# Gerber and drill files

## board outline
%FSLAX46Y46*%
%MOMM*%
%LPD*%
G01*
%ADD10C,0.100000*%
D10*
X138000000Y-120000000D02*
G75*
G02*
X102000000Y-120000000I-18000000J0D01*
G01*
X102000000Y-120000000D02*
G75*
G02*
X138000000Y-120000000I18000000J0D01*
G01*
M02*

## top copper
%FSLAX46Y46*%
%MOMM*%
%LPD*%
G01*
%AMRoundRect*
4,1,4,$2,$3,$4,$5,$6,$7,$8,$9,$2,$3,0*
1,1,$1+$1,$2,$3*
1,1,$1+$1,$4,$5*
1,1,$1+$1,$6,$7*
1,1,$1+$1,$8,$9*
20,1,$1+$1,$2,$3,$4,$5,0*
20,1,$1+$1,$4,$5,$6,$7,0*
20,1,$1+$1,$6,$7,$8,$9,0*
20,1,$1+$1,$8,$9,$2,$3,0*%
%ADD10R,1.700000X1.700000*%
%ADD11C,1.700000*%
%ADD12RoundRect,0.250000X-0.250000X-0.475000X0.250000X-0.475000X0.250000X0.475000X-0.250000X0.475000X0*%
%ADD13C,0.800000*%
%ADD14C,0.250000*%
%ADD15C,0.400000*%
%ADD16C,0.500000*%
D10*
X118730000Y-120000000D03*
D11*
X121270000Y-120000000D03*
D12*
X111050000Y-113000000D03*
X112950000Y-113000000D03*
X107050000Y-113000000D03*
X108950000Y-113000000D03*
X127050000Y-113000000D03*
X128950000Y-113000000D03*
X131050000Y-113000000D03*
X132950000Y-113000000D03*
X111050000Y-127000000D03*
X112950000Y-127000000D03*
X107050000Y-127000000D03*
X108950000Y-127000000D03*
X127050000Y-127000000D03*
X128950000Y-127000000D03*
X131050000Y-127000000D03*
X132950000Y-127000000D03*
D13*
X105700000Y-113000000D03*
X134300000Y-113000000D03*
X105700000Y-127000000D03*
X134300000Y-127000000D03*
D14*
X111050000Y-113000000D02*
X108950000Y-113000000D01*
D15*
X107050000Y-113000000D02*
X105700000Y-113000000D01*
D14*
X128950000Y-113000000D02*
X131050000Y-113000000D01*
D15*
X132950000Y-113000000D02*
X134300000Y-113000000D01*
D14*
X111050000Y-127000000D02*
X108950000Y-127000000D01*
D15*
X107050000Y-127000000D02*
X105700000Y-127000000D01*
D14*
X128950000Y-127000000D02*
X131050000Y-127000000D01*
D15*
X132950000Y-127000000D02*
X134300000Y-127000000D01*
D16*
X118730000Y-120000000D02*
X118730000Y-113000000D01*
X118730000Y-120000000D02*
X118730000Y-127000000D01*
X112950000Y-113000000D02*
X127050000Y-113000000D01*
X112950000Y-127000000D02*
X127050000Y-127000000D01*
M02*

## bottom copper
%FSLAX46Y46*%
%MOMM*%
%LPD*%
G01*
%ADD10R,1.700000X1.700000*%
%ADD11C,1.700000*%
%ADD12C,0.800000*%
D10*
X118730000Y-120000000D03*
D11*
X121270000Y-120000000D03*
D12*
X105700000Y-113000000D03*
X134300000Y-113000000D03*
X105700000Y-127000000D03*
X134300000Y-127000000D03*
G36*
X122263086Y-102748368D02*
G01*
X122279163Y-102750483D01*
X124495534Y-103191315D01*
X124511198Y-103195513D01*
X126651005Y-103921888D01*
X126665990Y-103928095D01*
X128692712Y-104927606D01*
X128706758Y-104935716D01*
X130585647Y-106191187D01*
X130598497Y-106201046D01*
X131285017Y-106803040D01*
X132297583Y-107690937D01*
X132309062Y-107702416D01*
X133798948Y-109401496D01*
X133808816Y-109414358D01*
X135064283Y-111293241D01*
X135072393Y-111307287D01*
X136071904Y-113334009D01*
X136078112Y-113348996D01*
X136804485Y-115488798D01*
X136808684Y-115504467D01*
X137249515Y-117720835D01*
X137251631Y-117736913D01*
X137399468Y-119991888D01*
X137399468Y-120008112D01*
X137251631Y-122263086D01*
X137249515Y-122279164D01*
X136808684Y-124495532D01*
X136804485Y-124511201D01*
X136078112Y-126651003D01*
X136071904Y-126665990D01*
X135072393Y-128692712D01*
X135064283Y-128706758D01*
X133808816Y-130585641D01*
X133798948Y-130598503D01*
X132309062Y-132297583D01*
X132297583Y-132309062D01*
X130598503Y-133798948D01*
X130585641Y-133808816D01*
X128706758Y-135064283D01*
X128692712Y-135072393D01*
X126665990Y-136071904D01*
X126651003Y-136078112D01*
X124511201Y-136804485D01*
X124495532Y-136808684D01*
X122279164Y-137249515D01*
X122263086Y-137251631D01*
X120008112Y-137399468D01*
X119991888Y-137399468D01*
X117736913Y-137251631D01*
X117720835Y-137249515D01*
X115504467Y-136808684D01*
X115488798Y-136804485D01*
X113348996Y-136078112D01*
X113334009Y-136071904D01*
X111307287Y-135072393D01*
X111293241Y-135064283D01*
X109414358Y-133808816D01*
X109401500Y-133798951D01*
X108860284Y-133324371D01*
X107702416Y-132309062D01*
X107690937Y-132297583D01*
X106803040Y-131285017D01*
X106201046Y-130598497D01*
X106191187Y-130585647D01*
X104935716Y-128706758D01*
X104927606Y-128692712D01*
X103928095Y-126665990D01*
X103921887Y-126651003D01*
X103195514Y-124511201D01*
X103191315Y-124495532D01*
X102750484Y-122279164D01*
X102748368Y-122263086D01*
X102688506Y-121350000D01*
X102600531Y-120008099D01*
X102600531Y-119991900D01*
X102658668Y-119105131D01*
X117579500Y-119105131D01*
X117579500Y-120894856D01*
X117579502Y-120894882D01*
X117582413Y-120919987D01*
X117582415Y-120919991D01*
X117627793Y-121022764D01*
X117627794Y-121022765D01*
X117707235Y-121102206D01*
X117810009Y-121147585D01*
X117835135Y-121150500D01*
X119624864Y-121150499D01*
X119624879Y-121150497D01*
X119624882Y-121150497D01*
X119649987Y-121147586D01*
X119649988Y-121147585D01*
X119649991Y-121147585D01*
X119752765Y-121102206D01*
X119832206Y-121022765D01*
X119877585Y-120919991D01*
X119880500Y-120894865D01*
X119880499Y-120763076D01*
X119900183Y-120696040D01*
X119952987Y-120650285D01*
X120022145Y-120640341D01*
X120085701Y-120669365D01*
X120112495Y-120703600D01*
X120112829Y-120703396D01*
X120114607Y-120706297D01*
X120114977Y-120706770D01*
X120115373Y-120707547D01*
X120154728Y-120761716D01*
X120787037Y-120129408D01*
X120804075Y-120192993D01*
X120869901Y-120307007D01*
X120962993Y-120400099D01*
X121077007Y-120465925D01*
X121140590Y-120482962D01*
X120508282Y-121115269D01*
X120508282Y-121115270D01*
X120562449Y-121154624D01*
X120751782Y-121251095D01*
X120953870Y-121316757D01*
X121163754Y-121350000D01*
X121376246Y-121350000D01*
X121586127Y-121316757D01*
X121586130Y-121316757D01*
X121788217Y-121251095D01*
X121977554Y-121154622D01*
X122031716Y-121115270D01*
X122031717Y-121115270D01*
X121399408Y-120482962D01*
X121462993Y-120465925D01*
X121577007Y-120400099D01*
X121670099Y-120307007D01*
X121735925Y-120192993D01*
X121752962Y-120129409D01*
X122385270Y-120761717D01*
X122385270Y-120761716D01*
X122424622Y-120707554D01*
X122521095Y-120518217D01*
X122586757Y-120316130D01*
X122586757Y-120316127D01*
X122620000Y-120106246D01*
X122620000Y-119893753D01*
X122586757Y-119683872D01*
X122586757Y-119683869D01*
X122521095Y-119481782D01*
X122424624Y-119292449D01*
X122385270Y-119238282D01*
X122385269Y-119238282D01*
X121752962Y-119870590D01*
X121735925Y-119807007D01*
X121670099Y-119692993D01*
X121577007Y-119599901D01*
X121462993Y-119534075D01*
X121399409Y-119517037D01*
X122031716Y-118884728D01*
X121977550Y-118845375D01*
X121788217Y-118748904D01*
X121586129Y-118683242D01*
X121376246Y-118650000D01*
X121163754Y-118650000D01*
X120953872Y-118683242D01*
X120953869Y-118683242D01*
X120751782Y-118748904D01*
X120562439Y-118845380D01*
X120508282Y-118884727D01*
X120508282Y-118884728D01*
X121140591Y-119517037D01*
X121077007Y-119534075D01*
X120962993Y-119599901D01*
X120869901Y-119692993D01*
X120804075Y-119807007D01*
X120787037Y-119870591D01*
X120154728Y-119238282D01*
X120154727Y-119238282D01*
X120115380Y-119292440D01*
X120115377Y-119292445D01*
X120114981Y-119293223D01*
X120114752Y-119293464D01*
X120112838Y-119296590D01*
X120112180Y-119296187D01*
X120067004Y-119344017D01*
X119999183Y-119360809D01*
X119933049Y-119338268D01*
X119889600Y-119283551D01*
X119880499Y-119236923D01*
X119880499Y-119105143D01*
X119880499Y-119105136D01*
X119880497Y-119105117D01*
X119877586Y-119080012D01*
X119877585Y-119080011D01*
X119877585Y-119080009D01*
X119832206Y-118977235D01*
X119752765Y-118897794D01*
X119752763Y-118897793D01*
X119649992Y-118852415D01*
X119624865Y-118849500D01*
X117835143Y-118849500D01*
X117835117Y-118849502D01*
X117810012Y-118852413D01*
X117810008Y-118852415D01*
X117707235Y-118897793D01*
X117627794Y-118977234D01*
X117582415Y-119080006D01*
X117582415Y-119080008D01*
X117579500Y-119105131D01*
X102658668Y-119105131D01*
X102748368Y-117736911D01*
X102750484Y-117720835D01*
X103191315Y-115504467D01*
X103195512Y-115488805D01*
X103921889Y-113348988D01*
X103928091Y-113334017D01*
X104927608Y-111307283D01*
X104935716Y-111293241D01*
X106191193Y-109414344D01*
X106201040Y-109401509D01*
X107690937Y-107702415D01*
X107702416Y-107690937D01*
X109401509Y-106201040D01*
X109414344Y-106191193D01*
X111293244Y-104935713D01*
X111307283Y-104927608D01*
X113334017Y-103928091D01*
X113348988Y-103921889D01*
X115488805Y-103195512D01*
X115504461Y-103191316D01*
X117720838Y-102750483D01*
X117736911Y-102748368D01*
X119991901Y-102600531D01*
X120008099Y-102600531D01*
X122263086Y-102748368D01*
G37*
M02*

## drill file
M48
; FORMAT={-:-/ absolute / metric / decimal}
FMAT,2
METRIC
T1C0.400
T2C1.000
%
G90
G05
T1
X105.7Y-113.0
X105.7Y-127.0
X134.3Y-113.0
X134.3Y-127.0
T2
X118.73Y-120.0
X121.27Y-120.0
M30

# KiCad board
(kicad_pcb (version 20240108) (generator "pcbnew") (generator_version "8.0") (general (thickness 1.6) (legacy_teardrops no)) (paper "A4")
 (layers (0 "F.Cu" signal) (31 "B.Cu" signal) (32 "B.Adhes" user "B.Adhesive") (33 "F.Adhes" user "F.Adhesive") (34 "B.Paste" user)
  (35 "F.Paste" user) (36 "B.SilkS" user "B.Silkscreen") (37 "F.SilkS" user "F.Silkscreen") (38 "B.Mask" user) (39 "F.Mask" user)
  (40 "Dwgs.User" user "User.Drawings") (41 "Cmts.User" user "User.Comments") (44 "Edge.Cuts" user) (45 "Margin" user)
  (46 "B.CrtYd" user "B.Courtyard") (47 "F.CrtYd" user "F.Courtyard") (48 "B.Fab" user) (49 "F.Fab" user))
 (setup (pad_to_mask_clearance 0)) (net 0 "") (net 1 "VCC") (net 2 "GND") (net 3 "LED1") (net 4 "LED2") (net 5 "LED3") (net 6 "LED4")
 (gr_circle (center 120 120) (end 138 120) (stroke (width 0.1) (type default)) (fill none) (layer "Edge.Cuts"))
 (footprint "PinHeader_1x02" (layer "F.Cu") (at 118.73 120)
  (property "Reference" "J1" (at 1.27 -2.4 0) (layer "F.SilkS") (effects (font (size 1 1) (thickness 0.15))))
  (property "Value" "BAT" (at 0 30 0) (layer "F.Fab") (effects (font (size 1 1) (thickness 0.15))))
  (pad "1" thru_hole rect (at 0 0) (size 1.7 1.7) (drill 1) (layers "*.Cu" "*.Mask") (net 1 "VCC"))
  (pad "2" thru_hole circle (at 2.54 0) (size 1.7 1.7) (drill 1) (layers "*.Cu" "*.Mask") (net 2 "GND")))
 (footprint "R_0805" (layer "F.Cu") (at 112 113)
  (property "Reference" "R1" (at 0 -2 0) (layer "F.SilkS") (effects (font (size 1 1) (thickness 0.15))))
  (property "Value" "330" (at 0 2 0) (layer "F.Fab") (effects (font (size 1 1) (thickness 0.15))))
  (pad "1" smd roundrect (at -0.95 0) (size 1 1.45) (layers "F.Cu" "F.Paste" "F.Mask") (roundrect_rratio 0.25) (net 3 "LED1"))
  (pad "2" smd roundrect (at 0.95 0) (size 1 1.45) (layers "F.Cu" "F.Paste" "F.Mask") (roundrect_rratio 0.25) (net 1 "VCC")))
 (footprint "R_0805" (layer "F.Cu") (at 108 113)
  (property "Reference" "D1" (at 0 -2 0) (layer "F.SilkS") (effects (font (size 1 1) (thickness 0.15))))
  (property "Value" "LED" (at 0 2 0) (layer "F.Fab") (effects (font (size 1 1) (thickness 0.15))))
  (pad "1" smd roundrect (at -0.95 0) (size 1 1.45) (layers "F.Cu" "F.Paste" "F.Mask") (roundrect_rratio 0.25) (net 2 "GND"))
  (pad "2" smd roundrect (at 0.95 0) (size 1 1.45) (layers "F.Cu" "F.Paste" "F.Mask") (roundrect_rratio 0.25) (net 3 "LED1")))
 (segment (start 111.05 113) (end 108.95 113) (width 0.25) (layer "F.Cu") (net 3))
 (segment (start 107.05 113) (end 105.7 113) (width 0.4) (layer "F.Cu") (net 2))
 (via (at 105.7 113) (size 0.8) (drill 0.4) (layers "F.Cu" "B.Cu") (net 2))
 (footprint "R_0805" (layer "F.Cu") (at 128 113)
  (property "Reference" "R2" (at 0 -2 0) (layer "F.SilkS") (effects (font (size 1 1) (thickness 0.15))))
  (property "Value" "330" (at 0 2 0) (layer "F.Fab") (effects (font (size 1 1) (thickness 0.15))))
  (pad "1" smd roundrect (at -0.95 0) (size 1 1.45) (layers "F.Cu" "F.Paste" "F.Mask") (roundrect_rratio 0.25) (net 1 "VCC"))
  (pad "2" smd roundrect (at 0.95 0) (size 1 1.45) (layers "F.Cu" "F.Paste" "F.Mask") (roundrect_rratio 0.25) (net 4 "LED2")))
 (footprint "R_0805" (layer "F.Cu") (at 132 113)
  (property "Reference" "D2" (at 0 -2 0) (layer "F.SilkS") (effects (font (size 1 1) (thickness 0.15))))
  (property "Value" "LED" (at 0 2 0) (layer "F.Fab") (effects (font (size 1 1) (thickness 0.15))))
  (pad "1" smd roundrect (at -0.95 0) (size 1 1.45) (layers "F.Cu" "F.Paste" "F.Mask") (roundrect_rratio 0.25) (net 4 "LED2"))
  (pad "2" smd roundrect (at 0.95 0) (size 1 1.45) (layers "F.Cu" "F.Paste" "F.Mask") (roundrect_rratio 0.25) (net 2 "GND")))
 (segment (start 128.95 113) (end 131.05 113) (width 0.25) (layer "F.Cu") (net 4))
 (segment (start 132.95 113) (end 134.3 113) (width 0.4) (layer "F.Cu") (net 2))
 (via (at 134.3 113) (size 0.8) (drill 0.4) (layers "F.Cu" "B.Cu") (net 2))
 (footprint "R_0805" (layer "F.Cu") (at 112 127)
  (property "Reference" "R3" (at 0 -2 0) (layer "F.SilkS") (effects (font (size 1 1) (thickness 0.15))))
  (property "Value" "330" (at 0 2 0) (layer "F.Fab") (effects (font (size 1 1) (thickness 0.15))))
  (pad "1" smd roundrect (at -0.95 0) (size 1 1.45) (layers "F.Cu" "F.Paste" "F.Mask") (roundrect_rratio 0.25) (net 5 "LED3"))
  (pad "2" smd roundrect (at 0.95 0) (size 1 1.45) (layers "F.Cu" "F.Paste" "F.Mask") (roundrect_rratio 0.25) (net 1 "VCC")))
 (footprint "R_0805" (layer "F.Cu") (at 108 127)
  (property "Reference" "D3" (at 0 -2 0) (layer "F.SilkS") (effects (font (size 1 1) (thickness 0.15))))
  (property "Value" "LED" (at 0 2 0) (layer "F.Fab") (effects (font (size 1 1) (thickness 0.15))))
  (pad "1" smd roundrect (at -0.95 0) (size 1 1.45) (layers "F.Cu" "F.Paste" "F.Mask") (roundrect_rratio 0.25) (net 2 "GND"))
  (pad "2" smd roundrect (at 0.95 0) (size 1 1.45) (layers "F.Cu" "F.Paste" "F.Mask") (roundrect_rratio 0.25) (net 5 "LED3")))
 (segment (start 111.05 127) (end 108.95 127) (width 0.25) (layer "F.Cu") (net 5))
 (segment (start 107.05 127) (end 105.7 127) (width 0.4) (layer "F.Cu") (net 2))
 (via (at 105.7 127) (size 0.8) (drill 0.4) (layers "F.Cu" "B.Cu") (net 2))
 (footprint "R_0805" (layer "F.Cu") (at 128 127)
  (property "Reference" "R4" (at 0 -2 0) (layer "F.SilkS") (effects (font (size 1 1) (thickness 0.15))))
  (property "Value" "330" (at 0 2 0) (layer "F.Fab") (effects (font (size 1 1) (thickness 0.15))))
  (pad "1" smd roundrect (at -0.95 0) (size 1 1.45) (layers "F.Cu" "F.Paste" "F.Mask") (roundrect_rratio 0.25) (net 1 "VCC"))
  (pad "2" smd roundrect (at 0.95 0) (size 1 1.45) (layers "F.Cu" "F.Paste" "F.Mask") (roundrect_rratio 0.25) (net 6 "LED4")))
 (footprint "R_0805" (layer "F.Cu") (at 132 127)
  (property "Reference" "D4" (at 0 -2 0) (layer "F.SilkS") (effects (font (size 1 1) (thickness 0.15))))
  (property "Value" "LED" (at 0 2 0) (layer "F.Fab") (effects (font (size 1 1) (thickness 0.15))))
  (pad "1" smd roundrect (at -0.95 0) (size 1 1.45) (layers "F.Cu" "F.Paste" "F.Mask") (roundrect_rratio 0.25) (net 6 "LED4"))
  (pad "2" smd roundrect (at 0.95 0) (size 1 1.45) (layers "F.Cu" "F.Paste" "F.Mask") (roundrect_rratio 0.25) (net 2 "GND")))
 (segment (start 128.95 127) (end 131.05 127) (width 0.25) (layer "F.Cu") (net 6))
 (segment (start 132.95 127) (end 134.3 127) (width 0.4) (layer "F.Cu") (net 2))
 (via (at 134.3 127) (size 0.8) (drill 0.4) (layers "F.Cu" "B.Cu") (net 2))
 (segment (start 118.73 120) (end 118.73 113) (width 0.5) (layer "F.Cu") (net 1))
 (segment (start 118.73 120) (end 118.73 127) (width 0.5) (layer "F.Cu") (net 1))
 (segment (start 112.95 113) (end 127.05 113) (width 0.5) (layer "F.Cu") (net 1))
 (segment (start 112.95 127) (end 127.05 127) (width 0.5) (layer "F.Cu") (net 1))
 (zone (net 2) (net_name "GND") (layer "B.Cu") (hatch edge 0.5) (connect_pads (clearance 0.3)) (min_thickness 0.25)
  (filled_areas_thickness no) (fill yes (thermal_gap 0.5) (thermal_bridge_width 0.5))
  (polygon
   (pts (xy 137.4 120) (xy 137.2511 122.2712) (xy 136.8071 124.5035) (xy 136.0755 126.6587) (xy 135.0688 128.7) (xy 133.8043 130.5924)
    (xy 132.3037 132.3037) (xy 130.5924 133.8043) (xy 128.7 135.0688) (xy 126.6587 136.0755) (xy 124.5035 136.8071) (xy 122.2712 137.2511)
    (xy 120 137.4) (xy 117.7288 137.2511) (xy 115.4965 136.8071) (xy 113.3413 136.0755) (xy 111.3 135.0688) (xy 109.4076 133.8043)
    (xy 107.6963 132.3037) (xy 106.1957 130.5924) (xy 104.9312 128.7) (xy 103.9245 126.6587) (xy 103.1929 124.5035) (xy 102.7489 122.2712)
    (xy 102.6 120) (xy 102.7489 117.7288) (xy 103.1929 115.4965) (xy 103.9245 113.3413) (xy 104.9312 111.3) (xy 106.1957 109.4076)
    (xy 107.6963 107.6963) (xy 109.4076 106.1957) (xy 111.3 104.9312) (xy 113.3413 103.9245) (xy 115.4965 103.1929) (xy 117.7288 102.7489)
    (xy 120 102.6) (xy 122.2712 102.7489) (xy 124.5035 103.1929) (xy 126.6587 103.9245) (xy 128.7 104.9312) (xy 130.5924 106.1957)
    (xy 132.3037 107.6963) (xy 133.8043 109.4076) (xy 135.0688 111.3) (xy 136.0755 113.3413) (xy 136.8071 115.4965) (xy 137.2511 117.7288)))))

